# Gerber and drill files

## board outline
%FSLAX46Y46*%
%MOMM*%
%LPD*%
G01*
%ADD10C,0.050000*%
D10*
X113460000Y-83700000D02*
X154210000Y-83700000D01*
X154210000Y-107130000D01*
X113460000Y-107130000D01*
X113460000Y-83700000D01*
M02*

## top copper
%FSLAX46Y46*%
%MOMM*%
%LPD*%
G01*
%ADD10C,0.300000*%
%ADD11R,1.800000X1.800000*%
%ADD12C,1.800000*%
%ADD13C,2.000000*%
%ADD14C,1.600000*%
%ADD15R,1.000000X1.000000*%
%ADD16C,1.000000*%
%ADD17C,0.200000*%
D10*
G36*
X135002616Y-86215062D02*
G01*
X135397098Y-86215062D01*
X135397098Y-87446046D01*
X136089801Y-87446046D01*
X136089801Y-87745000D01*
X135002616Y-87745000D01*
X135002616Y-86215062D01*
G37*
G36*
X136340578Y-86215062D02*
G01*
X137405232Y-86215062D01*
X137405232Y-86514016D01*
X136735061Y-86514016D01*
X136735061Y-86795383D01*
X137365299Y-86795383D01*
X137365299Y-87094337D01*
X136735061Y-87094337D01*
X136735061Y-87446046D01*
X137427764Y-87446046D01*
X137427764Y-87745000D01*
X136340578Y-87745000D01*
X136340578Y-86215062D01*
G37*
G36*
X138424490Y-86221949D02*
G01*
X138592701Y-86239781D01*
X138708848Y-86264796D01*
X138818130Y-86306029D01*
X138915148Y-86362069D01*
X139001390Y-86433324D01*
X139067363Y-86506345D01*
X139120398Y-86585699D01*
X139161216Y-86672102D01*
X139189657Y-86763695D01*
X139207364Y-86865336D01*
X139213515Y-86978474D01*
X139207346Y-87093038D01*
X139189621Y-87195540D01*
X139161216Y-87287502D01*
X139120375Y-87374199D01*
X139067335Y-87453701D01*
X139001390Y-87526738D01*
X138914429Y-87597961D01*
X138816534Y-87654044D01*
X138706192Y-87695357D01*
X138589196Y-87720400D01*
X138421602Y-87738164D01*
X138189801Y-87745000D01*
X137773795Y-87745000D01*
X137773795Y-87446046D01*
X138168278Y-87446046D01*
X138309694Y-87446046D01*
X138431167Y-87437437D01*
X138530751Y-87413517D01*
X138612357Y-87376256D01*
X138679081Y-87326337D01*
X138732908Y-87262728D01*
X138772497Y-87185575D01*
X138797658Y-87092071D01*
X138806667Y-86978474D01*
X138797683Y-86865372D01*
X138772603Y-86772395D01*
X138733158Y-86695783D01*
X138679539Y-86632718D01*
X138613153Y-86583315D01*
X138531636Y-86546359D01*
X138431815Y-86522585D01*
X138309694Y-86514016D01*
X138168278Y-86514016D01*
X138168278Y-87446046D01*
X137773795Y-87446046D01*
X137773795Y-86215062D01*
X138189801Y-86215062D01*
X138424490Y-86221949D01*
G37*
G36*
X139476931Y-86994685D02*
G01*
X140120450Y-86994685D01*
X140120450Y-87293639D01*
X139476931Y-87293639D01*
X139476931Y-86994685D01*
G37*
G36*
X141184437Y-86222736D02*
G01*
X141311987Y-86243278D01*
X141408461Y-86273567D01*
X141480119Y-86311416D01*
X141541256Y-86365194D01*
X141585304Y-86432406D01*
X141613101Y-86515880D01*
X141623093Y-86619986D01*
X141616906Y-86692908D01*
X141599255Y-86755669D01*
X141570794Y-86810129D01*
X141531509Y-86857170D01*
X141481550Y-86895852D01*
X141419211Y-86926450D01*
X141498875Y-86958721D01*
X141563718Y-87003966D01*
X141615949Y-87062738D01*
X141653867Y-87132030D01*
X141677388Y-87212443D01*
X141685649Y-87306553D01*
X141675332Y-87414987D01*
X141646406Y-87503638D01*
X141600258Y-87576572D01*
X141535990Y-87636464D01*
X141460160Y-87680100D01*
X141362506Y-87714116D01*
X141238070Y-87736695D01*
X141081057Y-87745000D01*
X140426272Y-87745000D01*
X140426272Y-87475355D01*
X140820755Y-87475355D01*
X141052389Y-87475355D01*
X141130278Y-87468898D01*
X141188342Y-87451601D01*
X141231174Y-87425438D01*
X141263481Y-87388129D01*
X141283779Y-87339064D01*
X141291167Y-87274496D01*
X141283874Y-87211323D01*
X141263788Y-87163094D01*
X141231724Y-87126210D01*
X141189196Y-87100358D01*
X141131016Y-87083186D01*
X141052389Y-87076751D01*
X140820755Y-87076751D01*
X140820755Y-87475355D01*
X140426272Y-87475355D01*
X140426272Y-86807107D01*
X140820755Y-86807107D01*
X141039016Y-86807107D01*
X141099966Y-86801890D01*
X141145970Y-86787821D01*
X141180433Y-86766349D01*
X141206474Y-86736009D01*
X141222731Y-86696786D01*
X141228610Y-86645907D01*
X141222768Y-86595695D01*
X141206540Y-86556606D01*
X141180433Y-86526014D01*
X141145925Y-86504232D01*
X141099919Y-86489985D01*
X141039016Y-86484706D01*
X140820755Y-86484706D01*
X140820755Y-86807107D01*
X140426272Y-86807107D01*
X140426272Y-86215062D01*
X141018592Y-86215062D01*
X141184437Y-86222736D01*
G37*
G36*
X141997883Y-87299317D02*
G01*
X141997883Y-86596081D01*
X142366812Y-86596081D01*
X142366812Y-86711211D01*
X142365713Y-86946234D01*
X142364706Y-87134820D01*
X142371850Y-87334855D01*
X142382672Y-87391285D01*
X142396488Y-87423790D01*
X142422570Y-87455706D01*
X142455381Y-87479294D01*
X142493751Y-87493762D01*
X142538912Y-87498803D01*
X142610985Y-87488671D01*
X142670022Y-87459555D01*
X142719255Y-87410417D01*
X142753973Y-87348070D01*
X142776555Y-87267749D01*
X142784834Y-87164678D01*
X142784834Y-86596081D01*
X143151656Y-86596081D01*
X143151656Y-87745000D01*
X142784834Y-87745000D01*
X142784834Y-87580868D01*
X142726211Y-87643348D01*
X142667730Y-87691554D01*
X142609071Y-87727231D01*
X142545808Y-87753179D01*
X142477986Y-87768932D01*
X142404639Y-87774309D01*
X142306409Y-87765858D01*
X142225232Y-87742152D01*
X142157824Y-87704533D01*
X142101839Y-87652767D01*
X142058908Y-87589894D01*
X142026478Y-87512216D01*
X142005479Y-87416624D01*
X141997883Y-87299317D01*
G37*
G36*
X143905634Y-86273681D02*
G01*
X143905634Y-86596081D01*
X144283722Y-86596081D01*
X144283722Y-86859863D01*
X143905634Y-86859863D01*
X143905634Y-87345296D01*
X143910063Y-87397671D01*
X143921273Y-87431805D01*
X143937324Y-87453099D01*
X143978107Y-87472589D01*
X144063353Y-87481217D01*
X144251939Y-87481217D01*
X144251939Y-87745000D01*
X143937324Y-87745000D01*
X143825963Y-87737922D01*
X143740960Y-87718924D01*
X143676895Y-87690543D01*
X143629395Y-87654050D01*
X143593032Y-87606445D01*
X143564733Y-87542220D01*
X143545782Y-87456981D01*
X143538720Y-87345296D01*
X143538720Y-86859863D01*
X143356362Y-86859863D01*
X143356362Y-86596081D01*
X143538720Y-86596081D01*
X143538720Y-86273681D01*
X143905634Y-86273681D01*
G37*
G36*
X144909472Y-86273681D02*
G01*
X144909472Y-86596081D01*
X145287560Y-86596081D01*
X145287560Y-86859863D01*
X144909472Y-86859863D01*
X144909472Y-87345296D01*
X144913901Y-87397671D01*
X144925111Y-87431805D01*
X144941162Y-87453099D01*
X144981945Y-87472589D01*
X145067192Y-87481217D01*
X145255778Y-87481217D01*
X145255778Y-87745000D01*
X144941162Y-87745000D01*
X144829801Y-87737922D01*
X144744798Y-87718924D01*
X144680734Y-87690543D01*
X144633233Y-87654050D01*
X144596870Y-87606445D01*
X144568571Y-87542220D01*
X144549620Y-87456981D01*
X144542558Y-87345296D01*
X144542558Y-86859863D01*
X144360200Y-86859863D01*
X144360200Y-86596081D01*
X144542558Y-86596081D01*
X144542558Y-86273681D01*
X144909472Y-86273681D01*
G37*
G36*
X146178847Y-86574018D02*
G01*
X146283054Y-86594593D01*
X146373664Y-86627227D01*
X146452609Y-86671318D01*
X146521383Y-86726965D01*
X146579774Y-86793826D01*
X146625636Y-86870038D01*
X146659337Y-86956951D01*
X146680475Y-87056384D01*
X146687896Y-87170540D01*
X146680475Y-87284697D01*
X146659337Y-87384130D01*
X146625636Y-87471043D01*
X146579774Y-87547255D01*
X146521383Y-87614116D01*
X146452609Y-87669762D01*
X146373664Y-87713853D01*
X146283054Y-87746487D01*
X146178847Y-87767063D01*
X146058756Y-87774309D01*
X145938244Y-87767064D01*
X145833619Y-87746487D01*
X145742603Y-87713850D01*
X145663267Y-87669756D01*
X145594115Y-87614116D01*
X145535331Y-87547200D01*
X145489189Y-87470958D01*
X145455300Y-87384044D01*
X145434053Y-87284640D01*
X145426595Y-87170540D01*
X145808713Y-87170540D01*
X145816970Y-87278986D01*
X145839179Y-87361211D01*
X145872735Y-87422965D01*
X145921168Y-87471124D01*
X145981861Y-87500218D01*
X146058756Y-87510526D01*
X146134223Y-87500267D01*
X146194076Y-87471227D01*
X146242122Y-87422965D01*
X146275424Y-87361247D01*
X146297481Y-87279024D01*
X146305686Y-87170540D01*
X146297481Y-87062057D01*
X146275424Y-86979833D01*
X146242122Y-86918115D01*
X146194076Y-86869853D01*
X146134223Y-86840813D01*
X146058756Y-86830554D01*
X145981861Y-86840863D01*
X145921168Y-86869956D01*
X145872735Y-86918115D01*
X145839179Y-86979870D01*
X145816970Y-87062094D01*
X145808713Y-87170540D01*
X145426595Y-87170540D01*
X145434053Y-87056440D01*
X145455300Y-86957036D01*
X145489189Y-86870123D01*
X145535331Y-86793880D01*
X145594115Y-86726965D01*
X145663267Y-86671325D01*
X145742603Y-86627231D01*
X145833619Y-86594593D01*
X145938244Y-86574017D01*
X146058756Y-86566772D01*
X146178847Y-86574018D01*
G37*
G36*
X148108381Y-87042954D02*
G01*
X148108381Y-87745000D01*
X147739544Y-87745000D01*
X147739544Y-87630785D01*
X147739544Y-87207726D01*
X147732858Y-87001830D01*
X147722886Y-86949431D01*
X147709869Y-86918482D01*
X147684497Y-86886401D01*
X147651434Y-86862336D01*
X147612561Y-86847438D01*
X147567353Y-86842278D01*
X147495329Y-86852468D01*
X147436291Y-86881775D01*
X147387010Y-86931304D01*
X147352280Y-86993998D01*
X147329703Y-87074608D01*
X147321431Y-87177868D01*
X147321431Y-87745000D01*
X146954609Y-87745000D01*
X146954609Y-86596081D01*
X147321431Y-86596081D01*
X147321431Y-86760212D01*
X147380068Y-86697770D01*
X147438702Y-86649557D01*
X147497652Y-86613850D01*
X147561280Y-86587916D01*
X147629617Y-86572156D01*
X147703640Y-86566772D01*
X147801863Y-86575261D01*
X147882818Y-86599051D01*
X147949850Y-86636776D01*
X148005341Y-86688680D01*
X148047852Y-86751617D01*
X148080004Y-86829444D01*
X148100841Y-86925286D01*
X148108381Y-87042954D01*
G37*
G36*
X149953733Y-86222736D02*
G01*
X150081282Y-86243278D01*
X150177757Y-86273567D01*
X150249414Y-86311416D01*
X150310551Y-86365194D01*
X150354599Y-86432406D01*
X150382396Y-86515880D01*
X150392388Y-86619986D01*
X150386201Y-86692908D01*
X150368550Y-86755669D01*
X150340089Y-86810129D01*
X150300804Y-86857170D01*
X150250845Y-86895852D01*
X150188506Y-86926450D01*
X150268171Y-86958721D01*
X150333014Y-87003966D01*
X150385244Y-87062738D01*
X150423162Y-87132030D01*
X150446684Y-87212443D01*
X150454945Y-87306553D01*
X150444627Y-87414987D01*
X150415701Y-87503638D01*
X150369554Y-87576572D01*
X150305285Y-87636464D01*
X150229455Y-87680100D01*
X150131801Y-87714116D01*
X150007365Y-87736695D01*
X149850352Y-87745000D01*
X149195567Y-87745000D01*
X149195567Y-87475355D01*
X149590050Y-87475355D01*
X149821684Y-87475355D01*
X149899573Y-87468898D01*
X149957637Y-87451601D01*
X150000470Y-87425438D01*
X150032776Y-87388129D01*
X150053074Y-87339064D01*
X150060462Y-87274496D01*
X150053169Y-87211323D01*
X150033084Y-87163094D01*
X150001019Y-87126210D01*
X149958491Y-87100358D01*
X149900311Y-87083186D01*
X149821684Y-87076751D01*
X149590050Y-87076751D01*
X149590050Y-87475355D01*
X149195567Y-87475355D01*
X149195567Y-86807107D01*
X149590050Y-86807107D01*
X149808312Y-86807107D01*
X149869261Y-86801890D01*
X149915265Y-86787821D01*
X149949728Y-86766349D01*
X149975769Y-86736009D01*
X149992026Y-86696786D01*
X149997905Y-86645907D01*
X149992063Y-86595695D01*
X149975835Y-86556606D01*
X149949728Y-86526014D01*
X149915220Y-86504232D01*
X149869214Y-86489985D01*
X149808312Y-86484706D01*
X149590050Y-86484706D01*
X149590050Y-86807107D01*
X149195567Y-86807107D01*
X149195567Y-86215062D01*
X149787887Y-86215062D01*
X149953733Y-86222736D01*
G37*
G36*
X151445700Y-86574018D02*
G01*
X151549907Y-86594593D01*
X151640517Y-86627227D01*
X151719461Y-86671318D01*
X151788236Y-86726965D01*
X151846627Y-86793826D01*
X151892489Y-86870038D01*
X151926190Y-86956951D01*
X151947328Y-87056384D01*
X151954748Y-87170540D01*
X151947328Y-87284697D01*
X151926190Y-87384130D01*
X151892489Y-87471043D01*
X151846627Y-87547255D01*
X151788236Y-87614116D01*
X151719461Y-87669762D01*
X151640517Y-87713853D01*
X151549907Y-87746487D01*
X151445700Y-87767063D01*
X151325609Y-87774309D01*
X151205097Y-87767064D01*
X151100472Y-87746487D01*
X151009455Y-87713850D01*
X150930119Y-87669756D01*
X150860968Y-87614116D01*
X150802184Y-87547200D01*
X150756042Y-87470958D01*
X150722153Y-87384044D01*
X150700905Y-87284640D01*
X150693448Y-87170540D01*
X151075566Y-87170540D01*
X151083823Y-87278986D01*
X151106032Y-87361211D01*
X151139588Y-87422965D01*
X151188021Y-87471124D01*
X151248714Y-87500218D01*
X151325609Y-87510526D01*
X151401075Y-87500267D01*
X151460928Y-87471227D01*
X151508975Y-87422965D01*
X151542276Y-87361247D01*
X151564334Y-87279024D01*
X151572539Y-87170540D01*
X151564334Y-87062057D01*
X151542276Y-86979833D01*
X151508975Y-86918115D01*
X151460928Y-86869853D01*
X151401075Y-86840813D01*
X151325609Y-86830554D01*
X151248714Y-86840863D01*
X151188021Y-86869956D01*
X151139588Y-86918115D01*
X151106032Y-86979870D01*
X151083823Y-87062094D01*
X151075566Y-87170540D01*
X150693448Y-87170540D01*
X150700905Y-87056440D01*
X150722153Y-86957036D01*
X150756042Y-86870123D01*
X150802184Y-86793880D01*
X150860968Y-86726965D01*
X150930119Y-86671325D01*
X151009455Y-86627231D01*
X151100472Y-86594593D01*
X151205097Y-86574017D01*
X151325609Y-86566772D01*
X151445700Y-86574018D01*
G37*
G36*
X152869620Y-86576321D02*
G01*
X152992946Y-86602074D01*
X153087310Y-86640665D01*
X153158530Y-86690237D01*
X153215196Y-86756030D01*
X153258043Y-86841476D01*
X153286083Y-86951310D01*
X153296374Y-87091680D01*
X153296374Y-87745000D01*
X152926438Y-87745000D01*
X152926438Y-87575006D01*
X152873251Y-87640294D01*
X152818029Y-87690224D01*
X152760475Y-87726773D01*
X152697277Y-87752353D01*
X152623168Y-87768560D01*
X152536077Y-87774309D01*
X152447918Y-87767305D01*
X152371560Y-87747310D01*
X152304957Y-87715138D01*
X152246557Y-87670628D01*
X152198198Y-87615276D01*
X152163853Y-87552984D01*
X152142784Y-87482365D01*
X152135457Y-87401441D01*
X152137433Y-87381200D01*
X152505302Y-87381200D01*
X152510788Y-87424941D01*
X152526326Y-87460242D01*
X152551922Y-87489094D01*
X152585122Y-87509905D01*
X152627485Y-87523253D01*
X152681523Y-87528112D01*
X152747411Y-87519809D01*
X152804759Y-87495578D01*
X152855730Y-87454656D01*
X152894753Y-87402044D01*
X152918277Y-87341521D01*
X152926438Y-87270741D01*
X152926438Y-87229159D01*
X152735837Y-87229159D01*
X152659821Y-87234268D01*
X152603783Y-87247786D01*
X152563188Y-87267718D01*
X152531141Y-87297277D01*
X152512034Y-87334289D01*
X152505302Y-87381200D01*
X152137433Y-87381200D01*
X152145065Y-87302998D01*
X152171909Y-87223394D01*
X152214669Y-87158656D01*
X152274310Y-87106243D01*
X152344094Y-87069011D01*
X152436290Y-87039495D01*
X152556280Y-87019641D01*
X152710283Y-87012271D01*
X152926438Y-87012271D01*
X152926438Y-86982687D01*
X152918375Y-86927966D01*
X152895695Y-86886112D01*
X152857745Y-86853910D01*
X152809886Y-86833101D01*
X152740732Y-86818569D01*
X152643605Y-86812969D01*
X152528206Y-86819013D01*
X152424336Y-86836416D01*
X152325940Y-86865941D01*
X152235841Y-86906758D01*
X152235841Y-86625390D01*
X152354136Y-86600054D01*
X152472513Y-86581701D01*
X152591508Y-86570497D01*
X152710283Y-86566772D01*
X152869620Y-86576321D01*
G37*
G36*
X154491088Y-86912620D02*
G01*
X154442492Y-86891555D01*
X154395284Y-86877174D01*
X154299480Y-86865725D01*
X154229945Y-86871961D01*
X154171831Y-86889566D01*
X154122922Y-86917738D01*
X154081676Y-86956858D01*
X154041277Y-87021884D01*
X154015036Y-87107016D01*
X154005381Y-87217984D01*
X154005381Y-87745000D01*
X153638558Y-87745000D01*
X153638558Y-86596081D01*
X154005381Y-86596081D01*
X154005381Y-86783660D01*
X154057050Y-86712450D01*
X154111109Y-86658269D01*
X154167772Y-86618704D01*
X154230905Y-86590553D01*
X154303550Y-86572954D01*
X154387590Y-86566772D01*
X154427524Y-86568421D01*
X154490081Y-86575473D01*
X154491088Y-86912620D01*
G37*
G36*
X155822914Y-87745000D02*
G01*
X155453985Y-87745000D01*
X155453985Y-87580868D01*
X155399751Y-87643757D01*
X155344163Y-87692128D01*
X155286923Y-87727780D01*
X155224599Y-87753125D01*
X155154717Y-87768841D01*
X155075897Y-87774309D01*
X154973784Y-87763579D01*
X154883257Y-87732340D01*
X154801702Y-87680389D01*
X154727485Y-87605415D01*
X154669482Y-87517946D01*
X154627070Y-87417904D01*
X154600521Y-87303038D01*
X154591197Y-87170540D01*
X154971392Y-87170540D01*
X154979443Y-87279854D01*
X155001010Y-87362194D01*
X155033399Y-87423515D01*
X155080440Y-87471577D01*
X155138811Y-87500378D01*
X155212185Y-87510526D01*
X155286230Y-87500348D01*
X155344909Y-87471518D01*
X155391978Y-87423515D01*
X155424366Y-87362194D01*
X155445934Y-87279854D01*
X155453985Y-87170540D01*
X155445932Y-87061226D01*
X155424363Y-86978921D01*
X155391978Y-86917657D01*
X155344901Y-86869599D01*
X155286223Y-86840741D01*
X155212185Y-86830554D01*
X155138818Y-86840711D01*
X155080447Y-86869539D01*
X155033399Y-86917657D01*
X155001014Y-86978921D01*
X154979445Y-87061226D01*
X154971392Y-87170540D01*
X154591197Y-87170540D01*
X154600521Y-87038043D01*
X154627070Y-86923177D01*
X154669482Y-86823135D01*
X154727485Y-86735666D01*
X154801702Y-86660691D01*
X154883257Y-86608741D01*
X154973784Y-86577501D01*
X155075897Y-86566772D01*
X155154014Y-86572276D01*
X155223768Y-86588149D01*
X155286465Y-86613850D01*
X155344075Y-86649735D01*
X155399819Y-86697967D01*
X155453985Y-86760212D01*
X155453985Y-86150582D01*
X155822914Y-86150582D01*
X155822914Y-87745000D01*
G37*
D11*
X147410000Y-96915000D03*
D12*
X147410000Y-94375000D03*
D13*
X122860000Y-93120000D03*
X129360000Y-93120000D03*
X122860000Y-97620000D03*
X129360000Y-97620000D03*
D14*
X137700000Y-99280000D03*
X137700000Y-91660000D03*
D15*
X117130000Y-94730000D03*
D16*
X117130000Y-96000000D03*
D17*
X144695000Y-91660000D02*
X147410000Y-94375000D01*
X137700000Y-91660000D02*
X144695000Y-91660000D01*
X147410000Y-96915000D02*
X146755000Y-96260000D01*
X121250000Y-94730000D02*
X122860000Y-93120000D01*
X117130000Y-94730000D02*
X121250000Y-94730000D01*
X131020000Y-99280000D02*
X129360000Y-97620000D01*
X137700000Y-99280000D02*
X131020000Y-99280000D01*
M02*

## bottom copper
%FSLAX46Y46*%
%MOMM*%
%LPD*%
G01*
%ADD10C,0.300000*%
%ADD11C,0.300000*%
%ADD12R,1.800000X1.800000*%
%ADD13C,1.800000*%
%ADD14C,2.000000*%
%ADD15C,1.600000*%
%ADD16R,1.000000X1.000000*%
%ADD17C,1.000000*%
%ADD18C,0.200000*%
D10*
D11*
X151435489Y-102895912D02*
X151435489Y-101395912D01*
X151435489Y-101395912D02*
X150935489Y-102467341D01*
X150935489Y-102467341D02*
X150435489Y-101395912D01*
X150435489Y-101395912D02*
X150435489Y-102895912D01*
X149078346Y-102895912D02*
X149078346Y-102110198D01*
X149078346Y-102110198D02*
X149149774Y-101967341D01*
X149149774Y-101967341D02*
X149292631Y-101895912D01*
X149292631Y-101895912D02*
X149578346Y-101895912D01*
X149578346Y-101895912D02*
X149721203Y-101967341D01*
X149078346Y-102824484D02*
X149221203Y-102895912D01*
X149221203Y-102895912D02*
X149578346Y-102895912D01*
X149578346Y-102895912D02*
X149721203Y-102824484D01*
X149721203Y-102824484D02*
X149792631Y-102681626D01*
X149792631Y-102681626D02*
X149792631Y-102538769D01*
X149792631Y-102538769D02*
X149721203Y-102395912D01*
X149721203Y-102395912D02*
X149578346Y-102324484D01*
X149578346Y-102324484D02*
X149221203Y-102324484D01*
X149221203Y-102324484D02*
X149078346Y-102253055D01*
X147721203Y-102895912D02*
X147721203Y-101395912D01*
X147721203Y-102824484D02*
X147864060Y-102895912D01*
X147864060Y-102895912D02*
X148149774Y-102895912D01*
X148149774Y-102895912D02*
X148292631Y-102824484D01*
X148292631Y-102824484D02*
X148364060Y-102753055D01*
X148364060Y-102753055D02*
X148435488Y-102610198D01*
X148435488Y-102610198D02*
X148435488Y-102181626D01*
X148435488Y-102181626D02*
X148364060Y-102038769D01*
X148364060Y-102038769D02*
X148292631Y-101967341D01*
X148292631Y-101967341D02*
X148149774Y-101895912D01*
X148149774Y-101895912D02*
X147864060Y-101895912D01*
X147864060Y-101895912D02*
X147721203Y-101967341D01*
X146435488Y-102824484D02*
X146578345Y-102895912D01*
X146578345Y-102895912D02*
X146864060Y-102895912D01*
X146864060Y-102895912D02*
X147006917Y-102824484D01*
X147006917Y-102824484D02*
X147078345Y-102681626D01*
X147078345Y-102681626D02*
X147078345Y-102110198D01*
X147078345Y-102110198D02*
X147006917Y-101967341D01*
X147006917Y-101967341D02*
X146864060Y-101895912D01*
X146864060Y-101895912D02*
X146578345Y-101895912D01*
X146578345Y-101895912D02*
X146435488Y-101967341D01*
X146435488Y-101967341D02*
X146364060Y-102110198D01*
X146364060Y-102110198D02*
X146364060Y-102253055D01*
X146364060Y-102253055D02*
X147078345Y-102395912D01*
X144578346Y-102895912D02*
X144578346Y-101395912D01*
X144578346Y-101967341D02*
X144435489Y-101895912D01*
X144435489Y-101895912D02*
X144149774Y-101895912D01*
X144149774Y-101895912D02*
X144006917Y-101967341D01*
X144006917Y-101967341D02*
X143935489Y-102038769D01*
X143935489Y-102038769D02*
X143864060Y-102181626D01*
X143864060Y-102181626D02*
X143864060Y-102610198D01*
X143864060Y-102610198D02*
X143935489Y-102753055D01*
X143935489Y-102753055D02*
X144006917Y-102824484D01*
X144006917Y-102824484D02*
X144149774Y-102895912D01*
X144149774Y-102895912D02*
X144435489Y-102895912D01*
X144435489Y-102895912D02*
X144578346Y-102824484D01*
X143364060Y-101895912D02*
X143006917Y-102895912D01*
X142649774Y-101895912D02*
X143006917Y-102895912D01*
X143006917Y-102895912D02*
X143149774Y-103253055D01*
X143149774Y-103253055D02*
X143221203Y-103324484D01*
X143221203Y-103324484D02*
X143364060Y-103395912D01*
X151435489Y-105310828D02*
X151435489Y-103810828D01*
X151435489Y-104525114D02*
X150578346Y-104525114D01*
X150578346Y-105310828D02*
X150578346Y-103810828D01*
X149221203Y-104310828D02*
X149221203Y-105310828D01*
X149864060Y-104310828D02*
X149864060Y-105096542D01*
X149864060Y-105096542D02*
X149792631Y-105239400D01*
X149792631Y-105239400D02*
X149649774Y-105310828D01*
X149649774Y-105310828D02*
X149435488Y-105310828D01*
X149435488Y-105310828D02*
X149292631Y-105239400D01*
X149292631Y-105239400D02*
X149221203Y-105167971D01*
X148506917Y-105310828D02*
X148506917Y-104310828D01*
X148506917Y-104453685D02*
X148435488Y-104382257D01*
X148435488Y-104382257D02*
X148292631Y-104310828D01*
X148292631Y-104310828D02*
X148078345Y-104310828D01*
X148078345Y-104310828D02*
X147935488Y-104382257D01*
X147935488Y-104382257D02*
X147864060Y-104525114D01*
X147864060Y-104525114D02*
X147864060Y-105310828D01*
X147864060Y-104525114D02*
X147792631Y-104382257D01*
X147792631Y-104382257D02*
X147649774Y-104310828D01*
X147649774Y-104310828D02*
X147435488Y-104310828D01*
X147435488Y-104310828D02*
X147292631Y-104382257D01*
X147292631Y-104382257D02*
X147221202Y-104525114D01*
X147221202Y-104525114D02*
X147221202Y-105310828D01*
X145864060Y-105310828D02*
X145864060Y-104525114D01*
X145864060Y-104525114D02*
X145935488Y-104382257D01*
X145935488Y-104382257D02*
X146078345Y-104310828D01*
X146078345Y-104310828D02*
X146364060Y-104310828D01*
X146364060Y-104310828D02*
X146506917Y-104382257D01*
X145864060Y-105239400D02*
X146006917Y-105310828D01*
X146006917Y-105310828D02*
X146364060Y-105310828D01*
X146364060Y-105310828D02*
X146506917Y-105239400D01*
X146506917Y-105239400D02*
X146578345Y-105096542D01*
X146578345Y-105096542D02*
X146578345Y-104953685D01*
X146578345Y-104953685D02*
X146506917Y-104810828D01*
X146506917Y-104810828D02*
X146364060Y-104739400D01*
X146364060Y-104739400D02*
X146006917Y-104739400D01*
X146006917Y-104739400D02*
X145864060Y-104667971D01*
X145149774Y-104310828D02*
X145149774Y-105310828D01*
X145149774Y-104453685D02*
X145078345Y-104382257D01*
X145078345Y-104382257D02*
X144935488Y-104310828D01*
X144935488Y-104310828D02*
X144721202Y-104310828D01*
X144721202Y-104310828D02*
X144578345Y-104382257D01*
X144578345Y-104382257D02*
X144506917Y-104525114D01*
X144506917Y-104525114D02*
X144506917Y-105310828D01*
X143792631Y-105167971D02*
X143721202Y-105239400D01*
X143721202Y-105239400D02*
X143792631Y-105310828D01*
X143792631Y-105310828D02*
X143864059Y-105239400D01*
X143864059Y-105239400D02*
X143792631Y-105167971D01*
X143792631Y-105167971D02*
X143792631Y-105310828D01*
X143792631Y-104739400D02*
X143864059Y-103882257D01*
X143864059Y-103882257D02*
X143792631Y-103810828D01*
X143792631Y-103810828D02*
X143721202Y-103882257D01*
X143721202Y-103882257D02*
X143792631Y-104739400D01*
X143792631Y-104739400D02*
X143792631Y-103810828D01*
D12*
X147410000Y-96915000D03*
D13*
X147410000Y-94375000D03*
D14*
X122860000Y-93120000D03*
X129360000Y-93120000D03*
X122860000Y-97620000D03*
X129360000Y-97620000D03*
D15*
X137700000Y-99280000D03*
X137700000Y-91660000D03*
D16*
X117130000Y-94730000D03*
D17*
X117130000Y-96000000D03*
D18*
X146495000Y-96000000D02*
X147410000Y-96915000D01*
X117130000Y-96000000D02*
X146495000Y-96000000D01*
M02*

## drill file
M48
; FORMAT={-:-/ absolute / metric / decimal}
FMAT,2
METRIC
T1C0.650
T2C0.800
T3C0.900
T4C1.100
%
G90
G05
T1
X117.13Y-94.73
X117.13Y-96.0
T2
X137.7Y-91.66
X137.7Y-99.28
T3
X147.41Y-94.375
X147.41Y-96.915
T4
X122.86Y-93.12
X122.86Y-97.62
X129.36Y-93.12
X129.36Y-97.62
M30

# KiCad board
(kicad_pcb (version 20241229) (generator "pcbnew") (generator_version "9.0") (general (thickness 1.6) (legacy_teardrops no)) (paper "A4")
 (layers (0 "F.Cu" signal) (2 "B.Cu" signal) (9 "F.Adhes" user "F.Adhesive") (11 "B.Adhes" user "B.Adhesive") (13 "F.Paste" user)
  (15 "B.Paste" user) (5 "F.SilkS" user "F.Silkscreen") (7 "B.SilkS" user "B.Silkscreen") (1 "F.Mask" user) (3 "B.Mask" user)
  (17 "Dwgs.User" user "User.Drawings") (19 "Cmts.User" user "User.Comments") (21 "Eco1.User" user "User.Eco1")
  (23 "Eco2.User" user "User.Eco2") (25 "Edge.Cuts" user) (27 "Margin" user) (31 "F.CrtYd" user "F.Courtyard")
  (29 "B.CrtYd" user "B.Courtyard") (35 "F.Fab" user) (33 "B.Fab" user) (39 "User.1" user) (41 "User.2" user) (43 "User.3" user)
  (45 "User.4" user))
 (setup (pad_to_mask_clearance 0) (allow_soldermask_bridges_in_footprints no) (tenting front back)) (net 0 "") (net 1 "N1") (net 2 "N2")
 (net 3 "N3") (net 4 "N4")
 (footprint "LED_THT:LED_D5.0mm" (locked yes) (layer "F.Cu") (at 147.41 96.915 90)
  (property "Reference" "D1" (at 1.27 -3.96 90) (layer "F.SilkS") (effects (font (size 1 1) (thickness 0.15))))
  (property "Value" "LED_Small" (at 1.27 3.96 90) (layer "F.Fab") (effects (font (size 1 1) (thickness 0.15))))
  (pad "1" thru_hole rect (at 0 0 90) (size 1.8 1.8) (drill 0.9) (layers "*.Cu" "*.Mask") (remove_unused_layers no) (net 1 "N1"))
  (pad "2" thru_hole circle (at 2.54 0 90) (size 1.8 1.8) (drill 0.9) (layers "*.Cu" "*.Mask") (remove_unused_layers no) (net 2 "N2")))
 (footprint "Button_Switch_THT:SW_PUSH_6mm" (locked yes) (layer "F.Cu") (at 122.86 93.12)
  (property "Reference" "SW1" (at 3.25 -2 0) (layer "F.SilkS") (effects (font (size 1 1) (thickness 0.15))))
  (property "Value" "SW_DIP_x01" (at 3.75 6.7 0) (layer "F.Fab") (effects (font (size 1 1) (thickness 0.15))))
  (pad "1" thru_hole circle (at 0 0 90) (size 2 2) (drill 1.1) (layers "*.Cu" "*.Mask") (remove_unused_layers no) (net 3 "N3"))
  (pad "1" thru_hole circle (at 6.5 0 90) (size 2 2) (drill 1.1) (layers "*.Cu" "*.Mask") (remove_unused_layers no) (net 3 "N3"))
  (pad "2" thru_hole circle (at 0 4.5 90) (size 2 2) (drill 1.1) (layers "*.Cu" "*.Mask") (remove_unused_layers no) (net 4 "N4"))
  (pad "2" thru_hole circle (at 6.5 4.5 90) (size 2 2) (drill 1.1) (layers "*.Cu" "*.Mask") (remove_unused_layers no) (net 4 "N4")))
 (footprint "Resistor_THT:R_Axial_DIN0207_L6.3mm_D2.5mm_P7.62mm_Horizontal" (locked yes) (layer "F.Cu") (at 137.7 99.28 90)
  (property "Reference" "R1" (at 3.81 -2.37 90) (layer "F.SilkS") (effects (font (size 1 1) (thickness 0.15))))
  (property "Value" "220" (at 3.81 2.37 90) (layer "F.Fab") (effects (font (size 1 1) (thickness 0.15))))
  (pad "1" thru_hole circle (at 0 0 90) (size 1.6 1.6) (drill 0.8) (layers "*.Cu" "*.Mask") (remove_unused_layers no) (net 4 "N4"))
  (pad "2" thru_hole circle (at 7.62 0 90) (size 1.6 1.6) (drill 0.8) (layers "*.Cu" "*.Mask") (remove_unused_layers no) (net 2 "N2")))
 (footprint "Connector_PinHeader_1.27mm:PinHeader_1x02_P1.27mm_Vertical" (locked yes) (layer "F.Cu") (at 117.13 94.73)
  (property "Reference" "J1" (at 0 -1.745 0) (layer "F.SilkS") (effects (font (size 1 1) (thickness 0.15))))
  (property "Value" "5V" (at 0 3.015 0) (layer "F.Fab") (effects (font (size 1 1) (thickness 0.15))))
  (pad "1" thru_hole rect (at 0 0) (size 1 1) (drill 0.65) (layers "*.Cu" "*.Mask") (remove_unused_layers no) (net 3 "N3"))
  (pad "2" thru_hole circle (at 0 1.27) (size 1 1) (drill 0.65) (layers "*.Cu" "*.Mask") (remove_unused_layers no) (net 1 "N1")))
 (gr_rect (start 113.46 83.7) (end 154.21 107.13) (stroke (width 0.05) (type default)) (fill no) (locked yes) (layer "Edge.Cuts"))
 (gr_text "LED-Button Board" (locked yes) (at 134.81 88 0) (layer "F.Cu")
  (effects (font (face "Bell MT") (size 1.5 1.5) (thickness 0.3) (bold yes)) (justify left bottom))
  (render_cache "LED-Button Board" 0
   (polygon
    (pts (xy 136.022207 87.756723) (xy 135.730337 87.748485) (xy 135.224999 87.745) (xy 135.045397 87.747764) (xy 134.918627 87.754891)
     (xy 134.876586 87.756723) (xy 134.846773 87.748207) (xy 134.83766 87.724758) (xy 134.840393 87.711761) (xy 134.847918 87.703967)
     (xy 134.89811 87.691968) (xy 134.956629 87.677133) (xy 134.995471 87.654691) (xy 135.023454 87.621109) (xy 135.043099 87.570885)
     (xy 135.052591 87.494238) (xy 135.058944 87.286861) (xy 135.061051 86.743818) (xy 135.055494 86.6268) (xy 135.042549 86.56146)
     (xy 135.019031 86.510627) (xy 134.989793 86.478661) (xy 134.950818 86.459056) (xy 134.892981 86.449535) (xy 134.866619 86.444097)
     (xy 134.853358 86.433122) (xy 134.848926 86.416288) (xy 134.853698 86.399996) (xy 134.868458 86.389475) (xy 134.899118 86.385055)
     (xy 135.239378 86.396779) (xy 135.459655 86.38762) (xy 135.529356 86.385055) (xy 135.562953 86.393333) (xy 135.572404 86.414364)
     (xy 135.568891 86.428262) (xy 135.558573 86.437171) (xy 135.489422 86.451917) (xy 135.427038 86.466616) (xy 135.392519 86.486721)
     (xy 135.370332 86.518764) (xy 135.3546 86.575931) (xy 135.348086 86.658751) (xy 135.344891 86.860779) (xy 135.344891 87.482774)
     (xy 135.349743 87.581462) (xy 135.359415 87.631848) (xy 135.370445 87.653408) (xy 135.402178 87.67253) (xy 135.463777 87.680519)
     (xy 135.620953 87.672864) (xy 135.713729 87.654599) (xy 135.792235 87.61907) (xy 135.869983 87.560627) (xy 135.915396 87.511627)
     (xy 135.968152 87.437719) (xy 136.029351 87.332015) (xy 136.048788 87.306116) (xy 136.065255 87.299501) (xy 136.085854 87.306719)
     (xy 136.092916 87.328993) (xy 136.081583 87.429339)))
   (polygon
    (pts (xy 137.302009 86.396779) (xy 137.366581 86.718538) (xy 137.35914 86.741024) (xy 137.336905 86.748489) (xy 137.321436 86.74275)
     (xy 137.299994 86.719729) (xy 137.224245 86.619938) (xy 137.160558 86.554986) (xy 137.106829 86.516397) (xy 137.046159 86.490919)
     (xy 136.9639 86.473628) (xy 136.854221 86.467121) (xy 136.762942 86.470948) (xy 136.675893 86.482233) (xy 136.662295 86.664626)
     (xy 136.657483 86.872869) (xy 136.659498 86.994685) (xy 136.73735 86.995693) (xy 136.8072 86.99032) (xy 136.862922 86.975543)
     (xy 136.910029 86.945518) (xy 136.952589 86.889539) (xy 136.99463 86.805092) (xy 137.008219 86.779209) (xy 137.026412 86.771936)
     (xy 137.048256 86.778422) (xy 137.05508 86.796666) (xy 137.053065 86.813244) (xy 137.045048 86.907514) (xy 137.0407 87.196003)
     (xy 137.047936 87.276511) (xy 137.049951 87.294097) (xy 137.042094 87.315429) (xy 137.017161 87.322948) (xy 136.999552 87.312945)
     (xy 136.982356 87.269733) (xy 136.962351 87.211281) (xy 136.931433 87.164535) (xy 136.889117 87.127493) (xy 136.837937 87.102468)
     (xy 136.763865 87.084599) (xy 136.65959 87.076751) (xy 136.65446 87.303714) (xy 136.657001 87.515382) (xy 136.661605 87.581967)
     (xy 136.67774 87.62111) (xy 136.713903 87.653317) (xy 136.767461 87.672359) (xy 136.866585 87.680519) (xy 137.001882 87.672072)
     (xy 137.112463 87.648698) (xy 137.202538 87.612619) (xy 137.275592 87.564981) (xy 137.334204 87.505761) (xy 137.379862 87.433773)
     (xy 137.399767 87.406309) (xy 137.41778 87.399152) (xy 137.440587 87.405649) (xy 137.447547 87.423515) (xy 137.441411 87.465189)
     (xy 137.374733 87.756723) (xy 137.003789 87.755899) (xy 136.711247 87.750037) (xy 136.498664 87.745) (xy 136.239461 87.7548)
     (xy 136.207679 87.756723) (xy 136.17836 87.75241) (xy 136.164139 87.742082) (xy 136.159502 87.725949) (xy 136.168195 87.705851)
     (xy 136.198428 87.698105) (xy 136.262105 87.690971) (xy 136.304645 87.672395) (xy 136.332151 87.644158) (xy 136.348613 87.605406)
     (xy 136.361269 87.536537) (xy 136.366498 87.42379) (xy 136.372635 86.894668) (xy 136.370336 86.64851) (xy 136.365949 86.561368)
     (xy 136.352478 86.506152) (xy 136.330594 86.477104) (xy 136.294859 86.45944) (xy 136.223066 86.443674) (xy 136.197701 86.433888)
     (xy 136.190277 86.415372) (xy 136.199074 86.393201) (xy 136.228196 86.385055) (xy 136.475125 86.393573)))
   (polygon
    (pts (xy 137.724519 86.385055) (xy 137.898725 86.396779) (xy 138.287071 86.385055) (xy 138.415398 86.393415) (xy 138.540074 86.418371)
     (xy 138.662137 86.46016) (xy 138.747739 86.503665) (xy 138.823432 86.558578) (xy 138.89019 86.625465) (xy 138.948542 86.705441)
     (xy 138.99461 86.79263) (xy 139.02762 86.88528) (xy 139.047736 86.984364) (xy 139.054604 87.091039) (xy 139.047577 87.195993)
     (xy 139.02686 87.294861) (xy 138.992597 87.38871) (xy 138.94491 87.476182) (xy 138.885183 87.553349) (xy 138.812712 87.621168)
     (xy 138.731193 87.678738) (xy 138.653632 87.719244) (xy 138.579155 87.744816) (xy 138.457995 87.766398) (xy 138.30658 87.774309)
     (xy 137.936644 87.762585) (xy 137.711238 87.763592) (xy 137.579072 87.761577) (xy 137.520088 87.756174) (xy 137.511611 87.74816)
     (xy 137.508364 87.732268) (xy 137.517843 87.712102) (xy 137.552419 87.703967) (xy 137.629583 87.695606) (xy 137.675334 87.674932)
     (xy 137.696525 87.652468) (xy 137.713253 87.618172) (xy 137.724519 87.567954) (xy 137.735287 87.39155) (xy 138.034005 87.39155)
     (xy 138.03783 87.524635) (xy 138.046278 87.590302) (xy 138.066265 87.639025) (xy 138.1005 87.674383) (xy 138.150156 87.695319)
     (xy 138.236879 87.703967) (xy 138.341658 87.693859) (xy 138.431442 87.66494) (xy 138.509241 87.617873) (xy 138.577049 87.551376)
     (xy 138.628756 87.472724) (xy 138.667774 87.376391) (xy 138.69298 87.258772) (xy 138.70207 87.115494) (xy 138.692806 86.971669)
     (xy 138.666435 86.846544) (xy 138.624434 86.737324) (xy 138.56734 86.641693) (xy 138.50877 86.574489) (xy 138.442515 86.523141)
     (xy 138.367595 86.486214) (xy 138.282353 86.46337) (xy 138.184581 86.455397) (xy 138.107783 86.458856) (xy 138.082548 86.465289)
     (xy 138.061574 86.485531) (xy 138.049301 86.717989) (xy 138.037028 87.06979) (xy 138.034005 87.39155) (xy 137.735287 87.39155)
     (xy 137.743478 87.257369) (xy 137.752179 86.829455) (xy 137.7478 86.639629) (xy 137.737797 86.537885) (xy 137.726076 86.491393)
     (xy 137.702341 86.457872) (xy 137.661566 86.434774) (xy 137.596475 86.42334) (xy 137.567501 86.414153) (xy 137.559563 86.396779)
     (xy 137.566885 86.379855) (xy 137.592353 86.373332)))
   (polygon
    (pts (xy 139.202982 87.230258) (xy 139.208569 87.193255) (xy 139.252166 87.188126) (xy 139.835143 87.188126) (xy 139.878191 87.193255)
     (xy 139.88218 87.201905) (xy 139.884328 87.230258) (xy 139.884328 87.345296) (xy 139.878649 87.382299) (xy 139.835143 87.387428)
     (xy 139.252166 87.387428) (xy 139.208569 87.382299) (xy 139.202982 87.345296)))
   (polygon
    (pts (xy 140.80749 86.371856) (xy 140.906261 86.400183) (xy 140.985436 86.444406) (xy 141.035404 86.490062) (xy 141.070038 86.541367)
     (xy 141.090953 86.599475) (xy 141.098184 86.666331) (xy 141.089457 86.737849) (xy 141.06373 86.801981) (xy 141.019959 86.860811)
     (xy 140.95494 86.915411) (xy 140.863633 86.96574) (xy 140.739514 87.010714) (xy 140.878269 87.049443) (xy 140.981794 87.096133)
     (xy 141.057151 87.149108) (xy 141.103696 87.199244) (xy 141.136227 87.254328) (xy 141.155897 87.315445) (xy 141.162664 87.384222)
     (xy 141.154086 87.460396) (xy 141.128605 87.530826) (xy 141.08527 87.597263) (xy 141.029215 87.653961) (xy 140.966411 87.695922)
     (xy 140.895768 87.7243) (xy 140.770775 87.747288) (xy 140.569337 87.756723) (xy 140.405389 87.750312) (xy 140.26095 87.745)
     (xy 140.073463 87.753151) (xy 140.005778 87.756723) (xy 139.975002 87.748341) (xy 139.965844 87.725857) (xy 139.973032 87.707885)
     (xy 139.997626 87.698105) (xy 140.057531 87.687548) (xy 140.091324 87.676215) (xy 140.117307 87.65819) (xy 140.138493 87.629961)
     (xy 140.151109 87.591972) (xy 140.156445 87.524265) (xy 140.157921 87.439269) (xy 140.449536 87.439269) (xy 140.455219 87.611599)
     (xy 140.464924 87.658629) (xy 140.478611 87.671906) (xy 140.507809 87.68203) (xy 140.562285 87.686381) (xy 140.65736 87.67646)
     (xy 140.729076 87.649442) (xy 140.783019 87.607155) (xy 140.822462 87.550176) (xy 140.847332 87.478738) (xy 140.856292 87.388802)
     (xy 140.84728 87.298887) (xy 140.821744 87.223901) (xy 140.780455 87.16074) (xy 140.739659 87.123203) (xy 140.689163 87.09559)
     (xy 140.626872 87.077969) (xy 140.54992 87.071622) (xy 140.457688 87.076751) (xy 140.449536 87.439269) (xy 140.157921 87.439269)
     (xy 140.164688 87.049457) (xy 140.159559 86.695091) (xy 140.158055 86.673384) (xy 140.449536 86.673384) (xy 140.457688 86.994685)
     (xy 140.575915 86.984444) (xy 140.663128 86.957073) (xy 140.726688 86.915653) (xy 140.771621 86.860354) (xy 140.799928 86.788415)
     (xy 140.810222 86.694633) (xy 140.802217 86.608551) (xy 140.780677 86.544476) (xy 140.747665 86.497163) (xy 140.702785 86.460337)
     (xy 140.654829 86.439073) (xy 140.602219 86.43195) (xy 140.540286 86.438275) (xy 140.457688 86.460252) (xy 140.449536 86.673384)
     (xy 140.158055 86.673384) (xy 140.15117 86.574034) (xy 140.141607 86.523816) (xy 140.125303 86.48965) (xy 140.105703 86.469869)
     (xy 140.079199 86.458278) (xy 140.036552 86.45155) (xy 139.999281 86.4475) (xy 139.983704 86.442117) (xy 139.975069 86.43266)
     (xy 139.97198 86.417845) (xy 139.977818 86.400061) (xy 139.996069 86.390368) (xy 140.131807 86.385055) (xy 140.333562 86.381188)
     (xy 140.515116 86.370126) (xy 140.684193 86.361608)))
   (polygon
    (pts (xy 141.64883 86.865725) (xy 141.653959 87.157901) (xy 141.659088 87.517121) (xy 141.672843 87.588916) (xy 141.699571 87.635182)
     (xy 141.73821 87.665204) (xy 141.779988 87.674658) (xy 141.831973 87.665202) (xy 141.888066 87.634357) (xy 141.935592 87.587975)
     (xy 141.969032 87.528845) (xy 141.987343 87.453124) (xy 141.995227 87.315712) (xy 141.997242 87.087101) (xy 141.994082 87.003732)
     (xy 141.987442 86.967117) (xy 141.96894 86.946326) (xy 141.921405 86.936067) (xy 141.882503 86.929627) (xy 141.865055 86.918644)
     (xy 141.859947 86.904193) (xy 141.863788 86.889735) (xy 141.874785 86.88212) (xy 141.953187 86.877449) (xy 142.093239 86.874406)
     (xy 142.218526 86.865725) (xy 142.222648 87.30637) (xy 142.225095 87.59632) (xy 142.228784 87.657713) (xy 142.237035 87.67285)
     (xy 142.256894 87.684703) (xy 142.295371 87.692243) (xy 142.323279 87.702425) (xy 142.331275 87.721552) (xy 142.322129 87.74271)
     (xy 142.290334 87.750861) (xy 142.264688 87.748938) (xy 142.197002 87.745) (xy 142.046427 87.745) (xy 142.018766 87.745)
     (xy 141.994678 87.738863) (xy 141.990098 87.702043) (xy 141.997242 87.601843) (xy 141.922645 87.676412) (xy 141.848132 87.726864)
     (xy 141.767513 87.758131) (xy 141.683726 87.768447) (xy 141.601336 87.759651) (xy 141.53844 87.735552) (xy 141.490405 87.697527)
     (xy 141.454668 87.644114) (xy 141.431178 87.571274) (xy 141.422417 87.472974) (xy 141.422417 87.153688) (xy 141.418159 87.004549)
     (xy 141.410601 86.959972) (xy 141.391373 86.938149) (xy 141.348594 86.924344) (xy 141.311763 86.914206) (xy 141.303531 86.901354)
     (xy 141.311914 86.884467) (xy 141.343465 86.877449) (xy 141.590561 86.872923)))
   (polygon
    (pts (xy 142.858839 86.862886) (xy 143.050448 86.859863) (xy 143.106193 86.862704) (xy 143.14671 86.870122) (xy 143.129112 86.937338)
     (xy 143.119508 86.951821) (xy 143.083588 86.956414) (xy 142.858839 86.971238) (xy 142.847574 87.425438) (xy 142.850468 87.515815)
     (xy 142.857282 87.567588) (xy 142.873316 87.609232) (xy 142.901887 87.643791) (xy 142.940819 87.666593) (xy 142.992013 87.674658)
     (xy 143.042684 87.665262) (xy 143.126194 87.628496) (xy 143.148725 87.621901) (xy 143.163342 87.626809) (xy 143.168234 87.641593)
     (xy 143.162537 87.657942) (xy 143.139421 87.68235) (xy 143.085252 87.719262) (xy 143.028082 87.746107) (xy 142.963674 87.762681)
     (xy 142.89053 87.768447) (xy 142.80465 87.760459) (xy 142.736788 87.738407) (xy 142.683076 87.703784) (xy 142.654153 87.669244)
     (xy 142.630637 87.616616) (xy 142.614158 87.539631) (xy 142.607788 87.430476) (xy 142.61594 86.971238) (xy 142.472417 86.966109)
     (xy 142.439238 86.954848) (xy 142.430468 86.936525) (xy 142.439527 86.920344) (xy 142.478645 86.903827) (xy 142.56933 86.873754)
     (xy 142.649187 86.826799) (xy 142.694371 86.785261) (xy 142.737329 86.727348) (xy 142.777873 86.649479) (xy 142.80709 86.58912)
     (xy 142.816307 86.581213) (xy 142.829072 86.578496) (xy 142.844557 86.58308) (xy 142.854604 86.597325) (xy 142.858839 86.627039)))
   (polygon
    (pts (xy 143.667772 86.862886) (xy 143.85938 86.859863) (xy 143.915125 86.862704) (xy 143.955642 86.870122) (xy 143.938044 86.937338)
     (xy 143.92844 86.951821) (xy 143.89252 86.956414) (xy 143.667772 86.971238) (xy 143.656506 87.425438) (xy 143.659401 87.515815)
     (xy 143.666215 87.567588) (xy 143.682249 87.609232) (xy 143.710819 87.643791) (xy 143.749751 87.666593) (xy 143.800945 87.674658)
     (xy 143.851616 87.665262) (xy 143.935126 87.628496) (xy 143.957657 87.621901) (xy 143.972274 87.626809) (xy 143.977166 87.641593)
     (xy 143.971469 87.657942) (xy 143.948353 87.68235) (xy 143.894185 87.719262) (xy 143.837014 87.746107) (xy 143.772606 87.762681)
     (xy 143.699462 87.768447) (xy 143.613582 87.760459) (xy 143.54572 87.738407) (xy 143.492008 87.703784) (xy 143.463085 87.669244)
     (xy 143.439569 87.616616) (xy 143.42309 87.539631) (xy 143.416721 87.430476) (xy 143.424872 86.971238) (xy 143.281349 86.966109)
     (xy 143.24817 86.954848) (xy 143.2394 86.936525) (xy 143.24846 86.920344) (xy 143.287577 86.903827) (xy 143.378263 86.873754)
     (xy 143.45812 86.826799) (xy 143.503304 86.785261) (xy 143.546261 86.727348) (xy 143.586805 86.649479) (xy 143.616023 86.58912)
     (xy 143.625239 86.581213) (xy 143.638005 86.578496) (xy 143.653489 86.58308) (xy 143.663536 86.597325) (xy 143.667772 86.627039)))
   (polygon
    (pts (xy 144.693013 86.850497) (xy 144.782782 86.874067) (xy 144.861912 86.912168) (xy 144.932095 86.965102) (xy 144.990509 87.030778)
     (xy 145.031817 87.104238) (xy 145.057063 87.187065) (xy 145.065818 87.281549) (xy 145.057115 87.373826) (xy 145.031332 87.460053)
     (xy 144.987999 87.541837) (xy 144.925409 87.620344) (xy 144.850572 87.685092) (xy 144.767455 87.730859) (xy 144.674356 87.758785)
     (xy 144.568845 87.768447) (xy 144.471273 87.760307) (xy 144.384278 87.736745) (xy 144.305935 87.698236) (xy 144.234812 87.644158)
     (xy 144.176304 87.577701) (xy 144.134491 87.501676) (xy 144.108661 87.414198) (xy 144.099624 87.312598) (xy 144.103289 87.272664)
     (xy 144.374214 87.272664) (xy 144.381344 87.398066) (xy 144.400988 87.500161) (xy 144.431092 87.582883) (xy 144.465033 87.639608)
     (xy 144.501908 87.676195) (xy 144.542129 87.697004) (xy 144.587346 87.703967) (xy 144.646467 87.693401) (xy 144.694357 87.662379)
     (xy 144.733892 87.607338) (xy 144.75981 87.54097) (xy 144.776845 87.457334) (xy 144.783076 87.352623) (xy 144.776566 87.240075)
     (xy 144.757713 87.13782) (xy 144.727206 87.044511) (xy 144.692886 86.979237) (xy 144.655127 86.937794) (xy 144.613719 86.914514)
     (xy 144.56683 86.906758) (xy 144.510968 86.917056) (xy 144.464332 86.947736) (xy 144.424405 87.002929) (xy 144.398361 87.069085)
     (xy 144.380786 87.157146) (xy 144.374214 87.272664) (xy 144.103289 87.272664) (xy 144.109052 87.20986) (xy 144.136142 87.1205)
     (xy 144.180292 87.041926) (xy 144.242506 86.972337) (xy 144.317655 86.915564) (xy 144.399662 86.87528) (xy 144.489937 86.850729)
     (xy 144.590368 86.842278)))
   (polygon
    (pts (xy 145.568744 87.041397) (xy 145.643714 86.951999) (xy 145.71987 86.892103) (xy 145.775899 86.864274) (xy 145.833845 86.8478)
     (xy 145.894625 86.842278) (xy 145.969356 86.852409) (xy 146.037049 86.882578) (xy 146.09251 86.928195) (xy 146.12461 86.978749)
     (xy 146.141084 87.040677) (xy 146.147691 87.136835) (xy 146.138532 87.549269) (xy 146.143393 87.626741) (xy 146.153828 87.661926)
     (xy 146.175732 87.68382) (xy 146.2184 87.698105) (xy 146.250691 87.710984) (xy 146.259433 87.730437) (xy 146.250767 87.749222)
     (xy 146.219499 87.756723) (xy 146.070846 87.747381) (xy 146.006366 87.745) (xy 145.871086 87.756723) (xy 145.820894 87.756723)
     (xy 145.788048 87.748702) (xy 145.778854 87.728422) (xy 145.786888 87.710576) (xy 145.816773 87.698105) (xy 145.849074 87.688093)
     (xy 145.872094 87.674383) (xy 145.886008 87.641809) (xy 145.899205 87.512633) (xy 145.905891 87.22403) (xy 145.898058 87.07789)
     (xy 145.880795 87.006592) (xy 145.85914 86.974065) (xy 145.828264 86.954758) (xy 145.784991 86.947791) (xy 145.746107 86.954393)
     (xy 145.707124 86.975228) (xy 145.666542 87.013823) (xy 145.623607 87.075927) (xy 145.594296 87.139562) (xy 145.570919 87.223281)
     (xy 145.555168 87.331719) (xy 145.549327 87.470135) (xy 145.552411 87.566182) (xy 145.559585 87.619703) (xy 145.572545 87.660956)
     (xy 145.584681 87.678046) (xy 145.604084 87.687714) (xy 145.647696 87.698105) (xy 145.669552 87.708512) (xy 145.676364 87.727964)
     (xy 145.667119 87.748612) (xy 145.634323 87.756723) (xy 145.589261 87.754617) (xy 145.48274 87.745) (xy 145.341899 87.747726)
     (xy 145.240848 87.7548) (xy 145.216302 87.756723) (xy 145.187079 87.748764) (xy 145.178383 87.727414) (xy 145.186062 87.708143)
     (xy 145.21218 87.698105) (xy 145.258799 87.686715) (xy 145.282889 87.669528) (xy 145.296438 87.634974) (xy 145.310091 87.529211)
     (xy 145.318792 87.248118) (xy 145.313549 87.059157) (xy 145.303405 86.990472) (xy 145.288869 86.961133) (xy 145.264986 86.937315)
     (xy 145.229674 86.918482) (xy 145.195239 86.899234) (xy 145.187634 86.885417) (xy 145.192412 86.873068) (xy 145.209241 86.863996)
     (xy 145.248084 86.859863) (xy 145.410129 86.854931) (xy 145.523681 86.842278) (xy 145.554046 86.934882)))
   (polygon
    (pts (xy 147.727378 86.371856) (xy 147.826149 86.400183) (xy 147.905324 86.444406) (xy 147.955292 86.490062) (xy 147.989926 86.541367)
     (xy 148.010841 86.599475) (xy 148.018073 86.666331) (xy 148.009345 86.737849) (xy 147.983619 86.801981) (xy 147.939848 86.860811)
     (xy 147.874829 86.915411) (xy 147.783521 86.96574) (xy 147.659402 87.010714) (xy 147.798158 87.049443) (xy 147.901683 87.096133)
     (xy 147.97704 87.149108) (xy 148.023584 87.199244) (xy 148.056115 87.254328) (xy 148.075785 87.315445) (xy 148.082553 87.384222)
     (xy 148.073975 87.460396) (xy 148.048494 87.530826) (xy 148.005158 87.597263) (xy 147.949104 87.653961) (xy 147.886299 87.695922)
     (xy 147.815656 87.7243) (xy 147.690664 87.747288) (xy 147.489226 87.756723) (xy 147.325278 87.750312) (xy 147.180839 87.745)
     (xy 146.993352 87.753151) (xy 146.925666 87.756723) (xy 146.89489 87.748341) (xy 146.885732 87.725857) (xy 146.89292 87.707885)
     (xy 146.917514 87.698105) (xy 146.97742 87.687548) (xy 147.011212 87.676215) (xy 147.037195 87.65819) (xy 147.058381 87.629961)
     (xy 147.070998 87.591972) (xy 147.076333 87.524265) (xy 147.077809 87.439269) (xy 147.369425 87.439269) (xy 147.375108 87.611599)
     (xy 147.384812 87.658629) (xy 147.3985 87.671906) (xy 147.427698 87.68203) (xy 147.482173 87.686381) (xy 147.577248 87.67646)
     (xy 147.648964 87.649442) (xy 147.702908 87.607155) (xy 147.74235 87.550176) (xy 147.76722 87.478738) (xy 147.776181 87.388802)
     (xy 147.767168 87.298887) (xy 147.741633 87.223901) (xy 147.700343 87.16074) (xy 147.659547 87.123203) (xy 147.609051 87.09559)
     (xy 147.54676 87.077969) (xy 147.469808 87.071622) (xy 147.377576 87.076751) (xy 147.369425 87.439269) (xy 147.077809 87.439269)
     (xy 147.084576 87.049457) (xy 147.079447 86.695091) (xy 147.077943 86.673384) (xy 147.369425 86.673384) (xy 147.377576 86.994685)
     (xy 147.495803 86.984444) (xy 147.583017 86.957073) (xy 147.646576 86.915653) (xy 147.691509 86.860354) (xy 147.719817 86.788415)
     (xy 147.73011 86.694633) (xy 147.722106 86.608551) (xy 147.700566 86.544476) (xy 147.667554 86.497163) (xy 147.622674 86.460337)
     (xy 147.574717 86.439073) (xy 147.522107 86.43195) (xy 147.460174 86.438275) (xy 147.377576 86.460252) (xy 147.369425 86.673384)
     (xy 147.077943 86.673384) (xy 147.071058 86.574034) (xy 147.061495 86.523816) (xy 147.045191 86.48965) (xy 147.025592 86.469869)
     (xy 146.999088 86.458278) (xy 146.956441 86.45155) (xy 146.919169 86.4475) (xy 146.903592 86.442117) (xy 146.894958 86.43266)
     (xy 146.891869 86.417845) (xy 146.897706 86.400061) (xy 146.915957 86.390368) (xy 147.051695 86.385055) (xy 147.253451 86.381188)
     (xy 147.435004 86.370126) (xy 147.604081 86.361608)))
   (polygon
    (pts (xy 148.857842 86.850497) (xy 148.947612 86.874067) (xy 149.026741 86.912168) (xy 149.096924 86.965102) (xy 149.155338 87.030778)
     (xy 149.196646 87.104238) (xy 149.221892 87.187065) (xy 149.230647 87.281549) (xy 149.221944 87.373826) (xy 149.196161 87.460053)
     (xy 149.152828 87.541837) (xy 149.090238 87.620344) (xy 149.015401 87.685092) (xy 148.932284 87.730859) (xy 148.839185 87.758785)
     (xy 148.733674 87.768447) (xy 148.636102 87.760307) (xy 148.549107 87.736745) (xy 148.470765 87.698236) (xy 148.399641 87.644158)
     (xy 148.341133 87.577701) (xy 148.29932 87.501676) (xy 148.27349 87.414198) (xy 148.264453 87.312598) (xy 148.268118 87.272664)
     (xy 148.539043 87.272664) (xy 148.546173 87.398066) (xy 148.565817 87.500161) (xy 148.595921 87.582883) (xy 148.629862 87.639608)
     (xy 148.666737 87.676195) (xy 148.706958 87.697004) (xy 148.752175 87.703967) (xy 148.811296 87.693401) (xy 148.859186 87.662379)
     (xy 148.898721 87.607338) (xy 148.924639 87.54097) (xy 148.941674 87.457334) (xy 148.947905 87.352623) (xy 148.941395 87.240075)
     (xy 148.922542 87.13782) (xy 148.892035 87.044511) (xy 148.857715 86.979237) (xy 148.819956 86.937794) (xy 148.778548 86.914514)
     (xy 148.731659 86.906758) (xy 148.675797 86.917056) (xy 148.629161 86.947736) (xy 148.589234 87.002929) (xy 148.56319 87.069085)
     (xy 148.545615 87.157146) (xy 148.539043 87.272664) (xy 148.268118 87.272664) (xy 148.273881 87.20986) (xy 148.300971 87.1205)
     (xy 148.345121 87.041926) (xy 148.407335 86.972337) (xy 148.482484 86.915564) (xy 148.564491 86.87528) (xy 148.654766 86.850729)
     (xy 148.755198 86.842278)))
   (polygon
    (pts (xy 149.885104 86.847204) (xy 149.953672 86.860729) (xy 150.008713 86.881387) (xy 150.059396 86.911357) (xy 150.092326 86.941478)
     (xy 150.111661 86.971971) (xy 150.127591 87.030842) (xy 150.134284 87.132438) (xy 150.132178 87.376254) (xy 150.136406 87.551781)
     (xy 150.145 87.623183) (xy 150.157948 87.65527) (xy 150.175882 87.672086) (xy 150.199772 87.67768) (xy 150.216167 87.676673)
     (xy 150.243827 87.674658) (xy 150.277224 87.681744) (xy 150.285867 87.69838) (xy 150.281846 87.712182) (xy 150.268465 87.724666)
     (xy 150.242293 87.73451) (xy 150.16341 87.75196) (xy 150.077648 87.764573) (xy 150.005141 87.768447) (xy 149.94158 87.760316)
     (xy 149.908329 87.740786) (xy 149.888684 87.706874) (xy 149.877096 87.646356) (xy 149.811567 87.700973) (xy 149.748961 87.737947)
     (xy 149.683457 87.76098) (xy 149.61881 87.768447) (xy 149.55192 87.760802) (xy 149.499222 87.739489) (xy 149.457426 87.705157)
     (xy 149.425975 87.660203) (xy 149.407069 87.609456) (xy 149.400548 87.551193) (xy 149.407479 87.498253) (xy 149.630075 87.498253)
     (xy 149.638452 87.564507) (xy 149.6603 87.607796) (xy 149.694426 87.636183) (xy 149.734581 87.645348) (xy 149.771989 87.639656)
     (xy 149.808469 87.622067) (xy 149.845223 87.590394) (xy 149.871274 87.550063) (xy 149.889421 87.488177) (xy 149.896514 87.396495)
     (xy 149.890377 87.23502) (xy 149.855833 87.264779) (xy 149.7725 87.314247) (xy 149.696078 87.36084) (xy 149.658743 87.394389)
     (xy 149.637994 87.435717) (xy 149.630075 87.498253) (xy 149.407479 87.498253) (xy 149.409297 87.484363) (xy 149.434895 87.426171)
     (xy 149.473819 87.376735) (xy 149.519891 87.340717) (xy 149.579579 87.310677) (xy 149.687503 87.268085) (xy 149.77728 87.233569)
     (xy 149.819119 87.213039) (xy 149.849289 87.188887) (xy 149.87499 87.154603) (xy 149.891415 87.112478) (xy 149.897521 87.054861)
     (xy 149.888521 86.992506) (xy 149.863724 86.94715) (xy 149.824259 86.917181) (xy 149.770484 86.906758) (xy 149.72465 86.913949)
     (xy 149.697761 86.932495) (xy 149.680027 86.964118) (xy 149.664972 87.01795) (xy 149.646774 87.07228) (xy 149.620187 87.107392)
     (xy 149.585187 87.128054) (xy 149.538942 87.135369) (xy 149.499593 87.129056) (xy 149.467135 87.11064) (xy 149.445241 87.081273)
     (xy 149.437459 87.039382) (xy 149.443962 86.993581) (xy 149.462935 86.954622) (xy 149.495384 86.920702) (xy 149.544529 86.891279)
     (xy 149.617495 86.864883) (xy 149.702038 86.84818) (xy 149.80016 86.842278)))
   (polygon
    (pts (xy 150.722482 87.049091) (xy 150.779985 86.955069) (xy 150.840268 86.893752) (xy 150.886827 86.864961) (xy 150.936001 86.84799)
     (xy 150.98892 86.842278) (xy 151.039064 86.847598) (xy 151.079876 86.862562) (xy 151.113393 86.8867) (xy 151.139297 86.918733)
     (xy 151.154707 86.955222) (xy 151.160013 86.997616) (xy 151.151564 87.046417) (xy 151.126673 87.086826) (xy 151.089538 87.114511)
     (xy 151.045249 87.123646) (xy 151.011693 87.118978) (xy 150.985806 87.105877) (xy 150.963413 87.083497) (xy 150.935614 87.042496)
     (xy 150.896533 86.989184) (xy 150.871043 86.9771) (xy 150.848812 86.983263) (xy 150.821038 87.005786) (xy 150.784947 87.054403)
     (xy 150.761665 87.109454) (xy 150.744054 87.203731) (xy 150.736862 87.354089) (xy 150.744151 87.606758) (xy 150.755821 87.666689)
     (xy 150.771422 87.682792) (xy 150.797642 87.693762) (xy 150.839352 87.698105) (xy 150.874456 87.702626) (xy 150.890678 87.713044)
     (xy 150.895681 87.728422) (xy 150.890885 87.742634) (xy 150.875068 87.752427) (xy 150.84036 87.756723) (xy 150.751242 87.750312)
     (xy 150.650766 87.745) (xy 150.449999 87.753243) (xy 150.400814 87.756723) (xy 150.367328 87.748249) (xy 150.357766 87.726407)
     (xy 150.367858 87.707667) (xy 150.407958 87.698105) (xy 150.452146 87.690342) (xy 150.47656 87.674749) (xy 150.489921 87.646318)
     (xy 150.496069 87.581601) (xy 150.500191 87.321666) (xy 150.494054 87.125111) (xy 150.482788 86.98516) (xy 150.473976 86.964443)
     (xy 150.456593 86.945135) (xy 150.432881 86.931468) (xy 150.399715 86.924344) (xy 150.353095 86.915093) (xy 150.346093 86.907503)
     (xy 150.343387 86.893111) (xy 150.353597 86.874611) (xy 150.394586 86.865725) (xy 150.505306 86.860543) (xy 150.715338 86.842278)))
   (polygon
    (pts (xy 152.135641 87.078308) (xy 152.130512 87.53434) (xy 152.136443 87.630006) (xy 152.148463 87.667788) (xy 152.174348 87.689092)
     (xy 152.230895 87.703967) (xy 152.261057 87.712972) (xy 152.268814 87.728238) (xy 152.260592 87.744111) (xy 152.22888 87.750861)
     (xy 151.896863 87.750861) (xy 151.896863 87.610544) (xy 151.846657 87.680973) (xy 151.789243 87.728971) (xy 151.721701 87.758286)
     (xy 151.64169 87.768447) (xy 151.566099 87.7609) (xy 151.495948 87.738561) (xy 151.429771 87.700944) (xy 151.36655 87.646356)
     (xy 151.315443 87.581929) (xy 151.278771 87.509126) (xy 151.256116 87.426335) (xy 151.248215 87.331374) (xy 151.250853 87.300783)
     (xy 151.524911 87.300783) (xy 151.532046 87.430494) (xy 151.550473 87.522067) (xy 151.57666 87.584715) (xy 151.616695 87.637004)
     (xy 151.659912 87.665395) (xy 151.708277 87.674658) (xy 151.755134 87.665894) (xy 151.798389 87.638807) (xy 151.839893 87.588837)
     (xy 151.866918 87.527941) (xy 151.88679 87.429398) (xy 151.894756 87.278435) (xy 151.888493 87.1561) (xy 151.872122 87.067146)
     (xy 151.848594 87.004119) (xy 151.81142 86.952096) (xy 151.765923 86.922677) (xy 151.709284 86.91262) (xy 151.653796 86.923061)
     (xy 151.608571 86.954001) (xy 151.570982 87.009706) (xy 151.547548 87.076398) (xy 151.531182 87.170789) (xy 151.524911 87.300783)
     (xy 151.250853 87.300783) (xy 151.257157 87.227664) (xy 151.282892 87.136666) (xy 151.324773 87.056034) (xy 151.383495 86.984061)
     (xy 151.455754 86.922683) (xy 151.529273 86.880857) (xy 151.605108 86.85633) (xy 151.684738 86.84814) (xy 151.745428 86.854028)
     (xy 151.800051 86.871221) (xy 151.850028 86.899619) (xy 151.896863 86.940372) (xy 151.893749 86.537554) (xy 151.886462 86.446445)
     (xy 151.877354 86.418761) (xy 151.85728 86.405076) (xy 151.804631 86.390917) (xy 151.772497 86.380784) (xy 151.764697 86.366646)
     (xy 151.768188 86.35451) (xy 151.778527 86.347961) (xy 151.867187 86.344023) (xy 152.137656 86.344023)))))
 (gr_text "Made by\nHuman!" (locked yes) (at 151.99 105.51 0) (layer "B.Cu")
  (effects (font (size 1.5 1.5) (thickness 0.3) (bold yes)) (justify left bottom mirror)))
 (segment (start 144.695 91.66) (end 147.41 94.375) (width 0.2) (locked yes) (layer "F.Cu") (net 2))
 (segment (start 137.7 91.66) (end 144.695 91.66) (width 0.2) (locked yes) (layer "F.Cu") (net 2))
 (segment (start 147.41 96.915) (end 146.755 96.26) (width 0.2) (locked yes) (layer "F.Cu") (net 1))
 (segment (start 146.495 96) (end 147.41 96.915) (width 0.2) (locked yes) (layer "B.Cu") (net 1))
 (segment (start 117.13 96) (end 146.495 96) (width 0.2) (locked yes) (layer "B.Cu") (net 1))
 (segment (start 121.25 94.73) (end 122.86 93.12) (width 0.2) (locked yes) (layer "F.Cu") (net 3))
 (segment (start 117.13 94.73) (end 121.25 94.73) (width 0.2) (locked yes) (layer "F.Cu") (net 3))
 (segment (start 131.02 99.28) (end 129.36 97.62) (width 0.2) (locked yes) (layer "F.Cu") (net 4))
 (segment (start 137.7 99.28) (end 131.02 99.28) (width 0.2) (locked yes) (layer "F.Cu") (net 4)))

